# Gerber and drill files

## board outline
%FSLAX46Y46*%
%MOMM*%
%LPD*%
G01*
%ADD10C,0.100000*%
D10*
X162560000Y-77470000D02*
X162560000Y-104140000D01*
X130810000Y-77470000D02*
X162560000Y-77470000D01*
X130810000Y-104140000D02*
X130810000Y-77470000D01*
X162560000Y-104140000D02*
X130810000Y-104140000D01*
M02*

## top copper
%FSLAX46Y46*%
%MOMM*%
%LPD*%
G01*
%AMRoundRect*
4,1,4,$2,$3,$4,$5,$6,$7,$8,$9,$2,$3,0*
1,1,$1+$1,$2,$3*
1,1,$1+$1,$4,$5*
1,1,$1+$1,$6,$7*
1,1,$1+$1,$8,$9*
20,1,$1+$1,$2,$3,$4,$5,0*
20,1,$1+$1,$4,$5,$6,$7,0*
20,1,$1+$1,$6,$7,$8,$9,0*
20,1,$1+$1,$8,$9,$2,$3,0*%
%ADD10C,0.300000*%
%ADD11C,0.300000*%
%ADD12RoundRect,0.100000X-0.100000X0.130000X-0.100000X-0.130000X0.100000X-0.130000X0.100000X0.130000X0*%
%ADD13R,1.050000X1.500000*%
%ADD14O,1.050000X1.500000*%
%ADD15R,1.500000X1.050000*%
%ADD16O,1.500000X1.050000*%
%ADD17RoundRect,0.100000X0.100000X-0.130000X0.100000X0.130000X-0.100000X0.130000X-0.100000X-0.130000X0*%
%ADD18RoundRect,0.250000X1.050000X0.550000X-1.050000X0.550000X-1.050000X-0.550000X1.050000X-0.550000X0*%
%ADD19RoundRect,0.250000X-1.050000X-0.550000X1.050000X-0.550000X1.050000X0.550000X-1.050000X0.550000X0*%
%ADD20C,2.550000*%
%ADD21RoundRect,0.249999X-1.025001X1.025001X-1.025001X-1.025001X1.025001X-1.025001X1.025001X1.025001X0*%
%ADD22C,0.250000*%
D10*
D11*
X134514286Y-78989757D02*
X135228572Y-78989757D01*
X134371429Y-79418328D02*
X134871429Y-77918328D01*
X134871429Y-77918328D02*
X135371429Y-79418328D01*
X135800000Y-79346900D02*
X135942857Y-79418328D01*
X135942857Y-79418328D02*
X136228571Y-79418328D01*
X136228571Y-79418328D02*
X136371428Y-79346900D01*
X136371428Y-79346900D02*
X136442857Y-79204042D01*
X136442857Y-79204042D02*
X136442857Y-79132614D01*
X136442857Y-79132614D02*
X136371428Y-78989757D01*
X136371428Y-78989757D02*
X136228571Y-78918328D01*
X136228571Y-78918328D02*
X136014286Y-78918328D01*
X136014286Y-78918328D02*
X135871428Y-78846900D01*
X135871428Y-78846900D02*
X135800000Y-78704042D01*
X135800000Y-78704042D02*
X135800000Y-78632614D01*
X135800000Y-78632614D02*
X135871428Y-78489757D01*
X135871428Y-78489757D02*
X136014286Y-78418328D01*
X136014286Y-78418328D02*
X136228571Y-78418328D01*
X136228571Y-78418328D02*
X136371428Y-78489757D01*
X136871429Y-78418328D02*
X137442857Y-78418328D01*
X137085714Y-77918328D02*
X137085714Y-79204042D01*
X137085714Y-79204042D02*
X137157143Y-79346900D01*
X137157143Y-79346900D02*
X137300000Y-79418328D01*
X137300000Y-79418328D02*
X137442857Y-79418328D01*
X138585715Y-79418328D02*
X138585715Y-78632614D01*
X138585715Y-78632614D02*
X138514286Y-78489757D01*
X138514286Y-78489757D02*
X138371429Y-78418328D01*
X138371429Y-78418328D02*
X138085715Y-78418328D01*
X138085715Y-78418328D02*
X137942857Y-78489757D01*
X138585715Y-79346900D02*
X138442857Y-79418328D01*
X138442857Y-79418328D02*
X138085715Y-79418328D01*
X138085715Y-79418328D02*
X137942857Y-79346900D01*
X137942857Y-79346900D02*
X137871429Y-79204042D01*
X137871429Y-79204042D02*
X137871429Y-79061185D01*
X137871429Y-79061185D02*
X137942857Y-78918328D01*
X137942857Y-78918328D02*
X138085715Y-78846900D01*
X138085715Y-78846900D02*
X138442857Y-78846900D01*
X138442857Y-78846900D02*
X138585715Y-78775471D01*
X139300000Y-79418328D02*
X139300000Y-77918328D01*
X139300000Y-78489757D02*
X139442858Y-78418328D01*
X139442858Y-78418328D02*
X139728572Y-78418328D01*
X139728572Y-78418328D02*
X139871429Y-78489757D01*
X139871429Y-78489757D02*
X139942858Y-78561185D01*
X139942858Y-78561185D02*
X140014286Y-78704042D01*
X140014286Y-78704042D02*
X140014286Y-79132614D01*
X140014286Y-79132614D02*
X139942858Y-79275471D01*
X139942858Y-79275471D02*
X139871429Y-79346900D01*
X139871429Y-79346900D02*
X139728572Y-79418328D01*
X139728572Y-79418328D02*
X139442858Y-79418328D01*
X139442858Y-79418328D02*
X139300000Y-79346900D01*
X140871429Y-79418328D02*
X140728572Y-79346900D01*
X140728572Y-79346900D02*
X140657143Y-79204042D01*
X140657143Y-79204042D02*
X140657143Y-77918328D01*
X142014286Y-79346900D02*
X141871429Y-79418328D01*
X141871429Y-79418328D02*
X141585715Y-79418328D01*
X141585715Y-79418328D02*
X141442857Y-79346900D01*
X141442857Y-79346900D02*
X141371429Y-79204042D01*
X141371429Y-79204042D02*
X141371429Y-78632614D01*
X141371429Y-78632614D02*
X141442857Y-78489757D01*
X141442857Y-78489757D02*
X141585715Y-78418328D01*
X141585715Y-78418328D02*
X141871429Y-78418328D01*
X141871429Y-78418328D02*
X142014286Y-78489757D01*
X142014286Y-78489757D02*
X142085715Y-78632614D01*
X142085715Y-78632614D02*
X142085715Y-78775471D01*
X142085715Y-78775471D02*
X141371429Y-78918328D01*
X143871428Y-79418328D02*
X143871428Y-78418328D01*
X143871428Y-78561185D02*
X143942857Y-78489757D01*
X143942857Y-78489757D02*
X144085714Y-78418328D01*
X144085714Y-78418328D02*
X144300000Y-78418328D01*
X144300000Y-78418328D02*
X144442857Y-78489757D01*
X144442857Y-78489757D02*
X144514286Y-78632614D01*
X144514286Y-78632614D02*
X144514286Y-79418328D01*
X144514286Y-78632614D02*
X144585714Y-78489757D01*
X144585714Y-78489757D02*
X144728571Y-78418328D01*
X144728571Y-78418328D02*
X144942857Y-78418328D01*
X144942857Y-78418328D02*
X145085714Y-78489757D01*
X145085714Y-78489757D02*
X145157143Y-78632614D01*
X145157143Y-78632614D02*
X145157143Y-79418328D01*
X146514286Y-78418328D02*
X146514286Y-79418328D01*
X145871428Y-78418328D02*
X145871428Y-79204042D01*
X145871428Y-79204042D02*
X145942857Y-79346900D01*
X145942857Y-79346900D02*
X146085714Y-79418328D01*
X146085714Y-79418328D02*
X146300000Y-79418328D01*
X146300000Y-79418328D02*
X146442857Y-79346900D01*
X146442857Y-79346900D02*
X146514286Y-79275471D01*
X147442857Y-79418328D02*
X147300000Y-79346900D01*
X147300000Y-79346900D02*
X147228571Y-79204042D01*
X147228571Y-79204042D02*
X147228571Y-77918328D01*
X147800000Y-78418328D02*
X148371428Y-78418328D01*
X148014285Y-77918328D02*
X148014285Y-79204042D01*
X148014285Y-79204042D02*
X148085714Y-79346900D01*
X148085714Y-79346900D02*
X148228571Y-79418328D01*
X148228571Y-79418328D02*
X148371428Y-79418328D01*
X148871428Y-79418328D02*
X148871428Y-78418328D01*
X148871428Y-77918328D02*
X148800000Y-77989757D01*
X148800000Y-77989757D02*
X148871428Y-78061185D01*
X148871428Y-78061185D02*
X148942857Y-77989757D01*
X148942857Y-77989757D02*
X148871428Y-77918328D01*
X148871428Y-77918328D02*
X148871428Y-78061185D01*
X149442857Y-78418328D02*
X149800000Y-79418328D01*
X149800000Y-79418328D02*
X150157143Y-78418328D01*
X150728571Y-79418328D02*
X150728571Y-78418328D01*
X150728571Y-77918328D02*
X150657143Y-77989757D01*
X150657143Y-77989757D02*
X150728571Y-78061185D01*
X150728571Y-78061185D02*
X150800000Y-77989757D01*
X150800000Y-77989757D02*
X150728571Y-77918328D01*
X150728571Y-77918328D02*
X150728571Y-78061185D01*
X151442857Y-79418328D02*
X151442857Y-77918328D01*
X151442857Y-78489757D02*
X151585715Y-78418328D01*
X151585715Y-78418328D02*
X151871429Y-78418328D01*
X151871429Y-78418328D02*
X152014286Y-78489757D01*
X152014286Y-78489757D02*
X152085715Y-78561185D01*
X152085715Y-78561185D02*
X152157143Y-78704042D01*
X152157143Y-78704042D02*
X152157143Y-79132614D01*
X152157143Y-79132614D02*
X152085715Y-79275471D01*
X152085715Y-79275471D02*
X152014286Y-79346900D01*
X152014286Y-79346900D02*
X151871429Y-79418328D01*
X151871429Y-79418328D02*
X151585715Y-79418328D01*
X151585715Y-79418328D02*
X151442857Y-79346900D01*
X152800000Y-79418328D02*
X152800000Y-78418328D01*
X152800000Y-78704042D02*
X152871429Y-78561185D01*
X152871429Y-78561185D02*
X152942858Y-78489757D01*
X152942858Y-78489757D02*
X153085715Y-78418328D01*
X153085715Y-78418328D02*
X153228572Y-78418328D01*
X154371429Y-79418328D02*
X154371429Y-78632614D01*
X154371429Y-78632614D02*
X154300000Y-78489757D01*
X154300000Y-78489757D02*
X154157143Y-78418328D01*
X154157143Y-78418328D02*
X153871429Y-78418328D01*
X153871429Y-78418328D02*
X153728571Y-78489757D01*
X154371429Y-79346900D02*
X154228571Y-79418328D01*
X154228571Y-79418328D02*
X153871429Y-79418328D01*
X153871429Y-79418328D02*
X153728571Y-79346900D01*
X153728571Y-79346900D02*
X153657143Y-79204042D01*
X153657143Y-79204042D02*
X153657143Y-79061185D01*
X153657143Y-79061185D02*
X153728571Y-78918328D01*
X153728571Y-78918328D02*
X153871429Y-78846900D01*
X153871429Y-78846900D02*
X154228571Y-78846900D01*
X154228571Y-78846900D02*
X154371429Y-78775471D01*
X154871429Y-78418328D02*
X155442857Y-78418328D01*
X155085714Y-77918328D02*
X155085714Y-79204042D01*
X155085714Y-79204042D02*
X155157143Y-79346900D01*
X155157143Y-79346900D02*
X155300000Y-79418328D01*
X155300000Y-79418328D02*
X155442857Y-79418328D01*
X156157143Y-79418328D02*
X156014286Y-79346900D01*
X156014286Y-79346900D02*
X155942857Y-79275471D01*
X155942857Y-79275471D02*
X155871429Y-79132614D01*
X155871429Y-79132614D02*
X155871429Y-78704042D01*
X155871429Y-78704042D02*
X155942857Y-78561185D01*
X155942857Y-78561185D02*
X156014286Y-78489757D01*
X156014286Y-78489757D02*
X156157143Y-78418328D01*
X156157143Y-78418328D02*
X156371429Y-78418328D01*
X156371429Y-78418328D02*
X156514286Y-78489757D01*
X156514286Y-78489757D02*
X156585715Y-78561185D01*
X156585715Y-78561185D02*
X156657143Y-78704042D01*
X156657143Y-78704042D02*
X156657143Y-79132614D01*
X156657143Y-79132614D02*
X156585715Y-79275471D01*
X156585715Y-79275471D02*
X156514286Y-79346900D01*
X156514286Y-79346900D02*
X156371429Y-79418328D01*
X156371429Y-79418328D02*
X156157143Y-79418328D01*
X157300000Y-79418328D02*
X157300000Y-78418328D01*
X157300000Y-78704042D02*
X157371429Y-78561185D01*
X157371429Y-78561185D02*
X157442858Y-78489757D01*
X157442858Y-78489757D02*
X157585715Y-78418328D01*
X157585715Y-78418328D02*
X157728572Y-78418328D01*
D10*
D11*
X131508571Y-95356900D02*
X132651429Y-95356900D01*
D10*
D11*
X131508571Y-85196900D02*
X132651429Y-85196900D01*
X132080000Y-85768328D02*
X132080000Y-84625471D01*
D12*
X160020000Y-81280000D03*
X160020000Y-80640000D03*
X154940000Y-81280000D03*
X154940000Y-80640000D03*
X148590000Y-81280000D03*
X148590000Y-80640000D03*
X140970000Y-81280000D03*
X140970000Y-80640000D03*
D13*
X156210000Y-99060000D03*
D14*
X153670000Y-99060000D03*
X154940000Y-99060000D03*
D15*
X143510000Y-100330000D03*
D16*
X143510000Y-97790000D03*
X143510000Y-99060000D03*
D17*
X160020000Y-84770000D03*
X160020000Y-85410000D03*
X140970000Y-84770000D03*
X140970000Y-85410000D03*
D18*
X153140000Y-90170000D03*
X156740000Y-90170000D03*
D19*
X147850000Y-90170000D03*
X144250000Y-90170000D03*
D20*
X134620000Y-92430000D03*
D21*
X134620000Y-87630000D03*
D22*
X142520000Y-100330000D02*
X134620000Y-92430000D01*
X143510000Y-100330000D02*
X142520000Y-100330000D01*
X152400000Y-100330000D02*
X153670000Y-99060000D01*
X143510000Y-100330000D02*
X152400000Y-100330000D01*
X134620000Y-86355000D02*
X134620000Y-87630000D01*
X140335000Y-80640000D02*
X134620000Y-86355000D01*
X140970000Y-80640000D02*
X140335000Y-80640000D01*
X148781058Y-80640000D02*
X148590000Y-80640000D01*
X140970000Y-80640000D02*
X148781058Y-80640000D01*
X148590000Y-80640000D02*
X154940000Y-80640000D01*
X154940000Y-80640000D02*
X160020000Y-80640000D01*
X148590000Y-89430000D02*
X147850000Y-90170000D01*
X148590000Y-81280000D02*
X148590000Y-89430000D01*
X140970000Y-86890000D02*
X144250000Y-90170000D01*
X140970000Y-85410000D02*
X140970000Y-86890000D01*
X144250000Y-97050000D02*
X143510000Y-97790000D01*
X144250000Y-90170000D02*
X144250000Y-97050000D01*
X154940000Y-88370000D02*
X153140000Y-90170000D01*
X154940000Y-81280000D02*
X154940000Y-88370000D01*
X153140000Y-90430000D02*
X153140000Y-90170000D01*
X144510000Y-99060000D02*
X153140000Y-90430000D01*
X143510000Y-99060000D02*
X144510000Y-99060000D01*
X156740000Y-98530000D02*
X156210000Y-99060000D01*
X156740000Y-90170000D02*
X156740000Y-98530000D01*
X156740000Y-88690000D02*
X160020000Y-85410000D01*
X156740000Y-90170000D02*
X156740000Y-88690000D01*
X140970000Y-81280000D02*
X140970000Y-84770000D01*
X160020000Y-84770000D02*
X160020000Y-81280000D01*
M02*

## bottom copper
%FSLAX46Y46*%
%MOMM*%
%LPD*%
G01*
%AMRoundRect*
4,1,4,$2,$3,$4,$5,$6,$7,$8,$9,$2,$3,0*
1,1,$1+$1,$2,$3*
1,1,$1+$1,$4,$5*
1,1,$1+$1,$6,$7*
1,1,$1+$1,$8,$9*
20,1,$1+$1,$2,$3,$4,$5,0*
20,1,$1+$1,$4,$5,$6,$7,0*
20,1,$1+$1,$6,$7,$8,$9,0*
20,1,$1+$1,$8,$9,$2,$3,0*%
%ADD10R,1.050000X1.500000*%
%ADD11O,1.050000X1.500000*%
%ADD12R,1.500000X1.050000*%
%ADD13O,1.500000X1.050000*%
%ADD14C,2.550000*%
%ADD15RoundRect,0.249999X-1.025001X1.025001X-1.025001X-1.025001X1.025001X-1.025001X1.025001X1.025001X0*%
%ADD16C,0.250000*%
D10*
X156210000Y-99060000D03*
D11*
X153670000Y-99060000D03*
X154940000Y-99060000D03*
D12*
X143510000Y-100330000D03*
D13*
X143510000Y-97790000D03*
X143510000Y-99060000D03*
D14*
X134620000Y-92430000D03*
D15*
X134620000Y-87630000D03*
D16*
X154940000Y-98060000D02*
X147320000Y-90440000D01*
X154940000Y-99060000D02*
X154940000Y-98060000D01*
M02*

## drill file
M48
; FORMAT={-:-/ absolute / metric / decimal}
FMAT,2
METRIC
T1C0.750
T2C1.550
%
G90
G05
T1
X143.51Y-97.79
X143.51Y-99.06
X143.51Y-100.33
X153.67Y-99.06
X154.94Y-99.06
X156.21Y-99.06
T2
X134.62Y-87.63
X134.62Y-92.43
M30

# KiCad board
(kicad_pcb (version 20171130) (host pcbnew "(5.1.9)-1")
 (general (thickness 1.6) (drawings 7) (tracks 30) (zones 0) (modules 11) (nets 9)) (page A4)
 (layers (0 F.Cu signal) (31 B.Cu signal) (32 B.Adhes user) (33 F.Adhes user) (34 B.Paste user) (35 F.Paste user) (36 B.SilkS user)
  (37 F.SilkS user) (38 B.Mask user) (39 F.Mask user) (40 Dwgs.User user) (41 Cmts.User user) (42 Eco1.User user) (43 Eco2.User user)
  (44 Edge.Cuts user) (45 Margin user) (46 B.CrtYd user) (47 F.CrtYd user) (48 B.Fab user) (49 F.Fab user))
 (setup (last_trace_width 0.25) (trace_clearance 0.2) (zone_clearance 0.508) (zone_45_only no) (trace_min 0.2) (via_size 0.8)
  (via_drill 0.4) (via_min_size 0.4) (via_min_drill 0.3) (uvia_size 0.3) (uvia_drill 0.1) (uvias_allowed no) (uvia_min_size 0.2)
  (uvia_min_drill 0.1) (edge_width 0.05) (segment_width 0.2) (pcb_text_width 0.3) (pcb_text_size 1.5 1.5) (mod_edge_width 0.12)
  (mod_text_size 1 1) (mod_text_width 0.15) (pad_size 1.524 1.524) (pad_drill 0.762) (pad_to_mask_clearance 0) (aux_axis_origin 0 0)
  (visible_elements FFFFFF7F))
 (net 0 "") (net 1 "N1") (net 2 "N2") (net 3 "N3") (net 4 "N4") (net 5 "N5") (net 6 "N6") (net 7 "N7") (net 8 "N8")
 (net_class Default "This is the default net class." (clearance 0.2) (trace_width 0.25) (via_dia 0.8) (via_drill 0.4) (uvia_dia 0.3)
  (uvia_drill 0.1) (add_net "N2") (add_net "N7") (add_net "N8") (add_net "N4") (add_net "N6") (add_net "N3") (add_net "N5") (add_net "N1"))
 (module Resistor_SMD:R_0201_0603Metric (layer F.Cu) (at 160.02 80.96 270)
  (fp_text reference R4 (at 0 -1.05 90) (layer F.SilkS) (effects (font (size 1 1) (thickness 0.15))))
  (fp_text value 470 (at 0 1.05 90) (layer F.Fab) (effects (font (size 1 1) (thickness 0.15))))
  (pad 2 smd roundrect (at 0.32 0 270) (size 0.46 0.4) (layers F.Cu F.Mask) (roundrect_rratio 0.25) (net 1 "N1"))
  (pad 1 smd roundrect (at -0.32 0 270) (size 0.46 0.4) (layers F.Cu F.Mask) (roundrect_rratio 0.25) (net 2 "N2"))
  (pad "" smd roundrect (at 0.345 0 270) (size 0.318 0.36) (layers F.Paste) (roundrect_rratio 0.25))
  (pad "" smd roundrect (at -0.345 0 270) (size 0.318 0.36) (layers F.Paste) (roundrect_rratio 0.25)))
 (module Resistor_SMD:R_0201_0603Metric (layer F.Cu) (at 154.94 80.96 270)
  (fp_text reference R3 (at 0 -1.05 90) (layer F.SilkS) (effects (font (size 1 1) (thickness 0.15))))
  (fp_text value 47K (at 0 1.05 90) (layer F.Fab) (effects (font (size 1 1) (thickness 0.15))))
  (pad 2 smd roundrect (at 0.32 0 270) (size 0.46 0.4) (layers F.Cu F.Mask) (roundrect_rratio 0.25) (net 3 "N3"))
  (pad 1 smd roundrect (at -0.32 0 270) (size 0.46 0.4) (layers F.Cu F.Mask) (roundrect_rratio 0.25) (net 2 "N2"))
  (pad "" smd roundrect (at 0.345 0 270) (size 0.318 0.36) (layers F.Paste) (roundrect_rratio 0.25))
  (pad "" smd roundrect (at -0.345 0 270) (size 0.318 0.36) (layers F.Paste) (roundrect_rratio 0.25)))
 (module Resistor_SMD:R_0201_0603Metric (layer F.Cu) (at 148.59 80.96 270)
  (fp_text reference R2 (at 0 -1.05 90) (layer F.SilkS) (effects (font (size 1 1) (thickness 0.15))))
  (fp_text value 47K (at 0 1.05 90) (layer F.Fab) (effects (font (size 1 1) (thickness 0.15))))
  (pad 2 smd roundrect (at 0.32 0 270) (size 0.46 0.4) (layers F.Cu F.Mask) (roundrect_rratio 0.25) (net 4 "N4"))
  (pad 1 smd roundrect (at -0.32 0 270) (size 0.46 0.4) (layers F.Cu F.Mask) (roundrect_rratio 0.25) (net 2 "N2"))
  (pad "" smd roundrect (at 0.345 0 270) (size 0.318 0.36) (layers F.Paste) (roundrect_rratio 0.25))
  (pad "" smd roundrect (at -0.345 0 270) (size 0.318 0.36) (layers F.Paste) (roundrect_rratio 0.25)))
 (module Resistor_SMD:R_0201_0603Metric (layer F.Cu) (at 140.97 80.96 270)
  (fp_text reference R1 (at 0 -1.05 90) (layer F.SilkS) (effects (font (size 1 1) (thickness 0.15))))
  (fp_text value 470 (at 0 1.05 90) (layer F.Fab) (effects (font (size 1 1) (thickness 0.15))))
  (pad 2 smd roundrect (at 0.32 0 270) (size 0.46 0.4) (layers F.Cu F.Mask) (roundrect_rratio 0.25) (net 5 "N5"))
  (pad 1 smd roundrect (at -0.32 0 270) (size 0.46 0.4) (layers F.Cu F.Mask) (roundrect_rratio 0.25) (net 2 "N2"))
  (pad "" smd roundrect (at 0.345 0 270) (size 0.318 0.36) (layers F.Paste) (roundrect_rratio 0.25))
  (pad "" smd roundrect (at -0.345 0 270) (size 0.318 0.36) (layers F.Paste) (roundrect_rratio 0.25)))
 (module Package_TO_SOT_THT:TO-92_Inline (layer F.Cu) (at 156.21 99.06 180)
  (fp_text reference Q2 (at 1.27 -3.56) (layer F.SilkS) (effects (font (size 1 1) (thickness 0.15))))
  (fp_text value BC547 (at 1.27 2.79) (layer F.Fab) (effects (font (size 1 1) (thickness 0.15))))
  (pad 1 thru_hole rect (at 0 0 180) (size 1.05 1.5) (drill 0.75) (layers *.Cu *.Mask) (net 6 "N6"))
  (pad 3 thru_hole oval (at 2.54 0 180) (size 1.05 1.5) (drill 0.75) (layers *.Cu *.Mask) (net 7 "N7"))
  (pad 2 thru_hole oval (at 1.27 0 180) (size 1.05 1.5) (drill 0.75) (layers *.Cu *.Mask) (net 4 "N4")))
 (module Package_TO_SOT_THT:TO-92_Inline (layer F.Cu) (at 143.51 100.33 90)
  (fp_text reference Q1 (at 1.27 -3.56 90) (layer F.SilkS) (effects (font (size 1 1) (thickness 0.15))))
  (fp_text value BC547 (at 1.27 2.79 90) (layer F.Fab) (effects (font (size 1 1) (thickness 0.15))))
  (pad 1 thru_hole rect (at 0 0 90) (size 1.05 1.5) (drill 0.75) (layers *.Cu *.Mask) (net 7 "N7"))
  (pad 3 thru_hole oval (at 2.54 0 90) (size 1.05 1.5) (drill 0.75) (layers *.Cu *.Mask) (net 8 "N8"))
  (pad 2 thru_hole oval (at 1.27 0 90) (size 1.05 1.5) (drill 0.75) (layers *.Cu *.Mask) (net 3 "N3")))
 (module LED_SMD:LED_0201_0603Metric (layer F.Cu) (at 160.02 85.09 90)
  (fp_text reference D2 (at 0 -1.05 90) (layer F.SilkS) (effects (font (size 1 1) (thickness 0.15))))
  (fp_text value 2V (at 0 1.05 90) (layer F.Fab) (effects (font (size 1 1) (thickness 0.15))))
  (pad 2 smd roundrect (at 0.32 0 90) (size 0.46 0.4) (layers F.Cu F.Mask) (roundrect_rratio 0.25) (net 1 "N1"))
  (pad 1 smd roundrect (at -0.32 0 90) (size 0.46 0.4) (layers F.Cu F.Mask) (roundrect_rratio 0.25) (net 6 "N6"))
  (pad "" smd roundrect (at 0.345 0 90) (size 0.318 0.36) (layers F.Paste) (roundrect_rratio 0.25))
  (pad "" smd roundrect (at -0.345 0 90) (size 0.318 0.36) (layers F.Paste) (roundrect_rratio 0.25)))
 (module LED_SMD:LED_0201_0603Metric (layer F.Cu) (at 140.97 85.09 90)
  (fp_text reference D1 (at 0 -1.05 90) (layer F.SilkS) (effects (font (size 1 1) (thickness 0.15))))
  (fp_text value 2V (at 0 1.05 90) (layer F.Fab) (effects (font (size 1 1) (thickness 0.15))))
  (pad 2 smd roundrect (at 0.32 0 90) (size 0.46 0.4) (layers F.Cu F.Mask) (roundrect_rratio 0.25) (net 5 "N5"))
  (pad 1 smd roundrect (at -0.32 0 90) (size 0.46 0.4) (layers F.Cu F.Mask) (roundrect_rratio 0.25) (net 8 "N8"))
  (pad "" smd roundrect (at 0.345 0 90) (size 0.318 0.36) (layers F.Paste) (roundrect_rratio 0.25))
  (pad "" smd roundrect (at -0.345 0 90) (size 0.318 0.36) (layers F.Paste) (roundrect_rratio 0.25)))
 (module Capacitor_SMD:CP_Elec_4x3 (layer F.Cu) (at 154.94 90.17 180)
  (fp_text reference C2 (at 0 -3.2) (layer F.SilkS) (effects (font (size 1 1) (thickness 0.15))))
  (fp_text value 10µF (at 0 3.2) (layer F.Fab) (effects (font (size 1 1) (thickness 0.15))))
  (pad 2 smd roundrect (at 1.8 0 180) (size 2.6 1.6) (layers F.Cu F.Paste F.Mask) (roundrect_rratio 0.15625) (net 3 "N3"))
  (pad 1 smd roundrect (at -1.8 0 180) (size 2.6 1.6) (layers F.Cu F.Paste F.Mask) (roundrect_rratio 0.15625) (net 6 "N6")))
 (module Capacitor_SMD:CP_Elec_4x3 (layer F.Cu) (at 146.05 90.17)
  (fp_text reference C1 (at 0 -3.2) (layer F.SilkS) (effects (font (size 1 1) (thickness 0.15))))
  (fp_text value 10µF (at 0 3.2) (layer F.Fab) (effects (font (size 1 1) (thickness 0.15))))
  (pad 2 smd roundrect (at 1.8 0) (size 2.6 1.6) (layers F.Cu F.Paste F.Mask) (roundrect_rratio 0.15625) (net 4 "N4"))
  (pad 1 smd roundrect (at -1.8 0) (size 2.6 1.6) (layers F.Cu F.Paste F.Mask) (roundrect_rratio 0.15625) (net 8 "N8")))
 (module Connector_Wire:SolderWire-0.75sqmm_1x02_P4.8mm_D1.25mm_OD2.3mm (layer F.Cu) (at 134.62 87.63 270)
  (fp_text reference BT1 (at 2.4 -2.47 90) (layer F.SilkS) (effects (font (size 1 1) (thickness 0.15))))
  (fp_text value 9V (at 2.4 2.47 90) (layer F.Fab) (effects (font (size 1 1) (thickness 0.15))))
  (pad 2 thru_hole circle (at 4.8 0 270) (size 2.55 2.55) (drill 1.55) (layers *.Cu *.Mask) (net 7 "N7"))
  (pad 1 thru_hole roundrect (at 0 0 270) (size 2.55 2.55) (drill 1.55) (layers *.Cu *.Mask) (roundrect_rratio 0.098039) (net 2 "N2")))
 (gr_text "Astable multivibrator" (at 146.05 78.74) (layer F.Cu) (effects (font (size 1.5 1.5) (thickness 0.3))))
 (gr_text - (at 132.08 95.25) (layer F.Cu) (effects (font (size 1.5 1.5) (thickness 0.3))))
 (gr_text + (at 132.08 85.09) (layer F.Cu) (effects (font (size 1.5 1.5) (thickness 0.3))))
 (gr_line (start 162.56 77.47) (end 162.56 104.14) (layer Edge.Cuts) (width 0.1))
 (gr_line (start 130.81 77.47) (end 162.56 77.47) (layer Edge.Cuts) (width 0.1))
 (gr_line (start 130.81 104.14) (end 130.81 77.47) (layer Edge.Cuts) (width 0.1))
 (gr_line (start 162.56 104.14) (end 130.81 104.14) (layer Edge.Cuts) (width 0.1))
 (segment (start 142.52 100.33) (end 134.62 92.43) (width 0.25) (layer F.Cu) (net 7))
 (segment (start 143.51 100.33) (end 142.52 100.33) (width 0.25) (layer F.Cu) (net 7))
 (segment (start 152.4 100.33) (end 153.67 99.06) (width 0.25) (layer F.Cu) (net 7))
 (segment (start 143.51 100.33) (end 152.4 100.33) (width 0.25) (layer F.Cu) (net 7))
 (segment (start 134.62 86.355) (end 134.62 87.63) (width 0.25) (layer F.Cu) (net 2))
 (segment (start 140.335 80.64) (end 134.62 86.355) (width 0.25) (layer F.Cu) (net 2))
 (segment (start 140.97 80.64) (end 140.335 80.64) (width 0.25) (layer F.Cu) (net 2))
 (segment (start 148.781058 80.64) (end 148.59 80.64) (width 0.25) (layer F.Cu) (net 2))
 (segment (start 140.97 80.64) (end 148.781058 80.64) (width 0.25) (layer F.Cu) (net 2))
 (segment (start 148.59 80.64) (end 154.94 80.64) (width 0.25) (layer F.Cu) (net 2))
 (segment (start 154.94 80.64) (end 160.02 80.64) (width 0.25) (layer F.Cu) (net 2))
 (segment (start 148.59 89.43) (end 147.85 90.17) (width 0.25) (layer F.Cu) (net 4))
 (segment (start 148.59 81.28) (end 148.59 89.43) (width 0.25) (layer F.Cu) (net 4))
 (segment (start 154.94 98.06) (end 147.32 90.44) (width 0.25) (layer B.Cu) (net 4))
 (segment (start 154.94 99.06) (end 154.94 98.06) (width 0.25) (layer B.Cu) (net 4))
 (segment (start 140.97 86.89) (end 144.25 90.17) (width 0.25) (layer F.Cu) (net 8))
 (segment (start 140.97 85.41) (end 140.97 86.89) (width 0.25) (layer F.Cu) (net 8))
 (segment (start 144.25 97.05) (end 143.51 97.79) (width 0.25) (layer F.Cu) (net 8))
 (segment (start 144.25 90.17) (end 144.25 97.05) (width 0.25) (layer F.Cu) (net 8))
 (segment (start 154.94 88.37) (end 153.14 90.17) (width 0.25) (layer F.Cu) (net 3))
 (segment (start 154.94 81.28) (end 154.94 88.37) (width 0.25) (layer F.Cu) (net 3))
 (segment (start 153.14 90.43) (end 153.14 90.17) (width 0.25) (layer F.Cu) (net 3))
 (segment (start 144.51 99.06) (end 153.14 90.43) (width 0.25) (layer F.Cu) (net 3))
 (segment (start 143.51 99.06) (end 144.51 99.06) (width 0.25) (layer F.Cu) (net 3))
 (segment (start 156.74 98.53) (end 156.21 99.06) (width 0.25) (layer F.Cu) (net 6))
 (segment (start 156.74 90.17) (end 156.74 98.53) (width 0.25) (layer F.Cu) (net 6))
 (segment (start 156.74 88.69) (end 160.02 85.41) (width 0.25) (layer F.Cu) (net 6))
 (segment (start 156.74 90.17) (end 156.74 88.69) (width 0.25) (layer F.Cu) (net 6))
 (segment (start 140.97 81.28) (end 140.97 84.77) (width 0.25) (layer F.Cu) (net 5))
 (segment (start 160.02 84.77) (end 160.02 81.28) (width 0.25) (layer F.Cu) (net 1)))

